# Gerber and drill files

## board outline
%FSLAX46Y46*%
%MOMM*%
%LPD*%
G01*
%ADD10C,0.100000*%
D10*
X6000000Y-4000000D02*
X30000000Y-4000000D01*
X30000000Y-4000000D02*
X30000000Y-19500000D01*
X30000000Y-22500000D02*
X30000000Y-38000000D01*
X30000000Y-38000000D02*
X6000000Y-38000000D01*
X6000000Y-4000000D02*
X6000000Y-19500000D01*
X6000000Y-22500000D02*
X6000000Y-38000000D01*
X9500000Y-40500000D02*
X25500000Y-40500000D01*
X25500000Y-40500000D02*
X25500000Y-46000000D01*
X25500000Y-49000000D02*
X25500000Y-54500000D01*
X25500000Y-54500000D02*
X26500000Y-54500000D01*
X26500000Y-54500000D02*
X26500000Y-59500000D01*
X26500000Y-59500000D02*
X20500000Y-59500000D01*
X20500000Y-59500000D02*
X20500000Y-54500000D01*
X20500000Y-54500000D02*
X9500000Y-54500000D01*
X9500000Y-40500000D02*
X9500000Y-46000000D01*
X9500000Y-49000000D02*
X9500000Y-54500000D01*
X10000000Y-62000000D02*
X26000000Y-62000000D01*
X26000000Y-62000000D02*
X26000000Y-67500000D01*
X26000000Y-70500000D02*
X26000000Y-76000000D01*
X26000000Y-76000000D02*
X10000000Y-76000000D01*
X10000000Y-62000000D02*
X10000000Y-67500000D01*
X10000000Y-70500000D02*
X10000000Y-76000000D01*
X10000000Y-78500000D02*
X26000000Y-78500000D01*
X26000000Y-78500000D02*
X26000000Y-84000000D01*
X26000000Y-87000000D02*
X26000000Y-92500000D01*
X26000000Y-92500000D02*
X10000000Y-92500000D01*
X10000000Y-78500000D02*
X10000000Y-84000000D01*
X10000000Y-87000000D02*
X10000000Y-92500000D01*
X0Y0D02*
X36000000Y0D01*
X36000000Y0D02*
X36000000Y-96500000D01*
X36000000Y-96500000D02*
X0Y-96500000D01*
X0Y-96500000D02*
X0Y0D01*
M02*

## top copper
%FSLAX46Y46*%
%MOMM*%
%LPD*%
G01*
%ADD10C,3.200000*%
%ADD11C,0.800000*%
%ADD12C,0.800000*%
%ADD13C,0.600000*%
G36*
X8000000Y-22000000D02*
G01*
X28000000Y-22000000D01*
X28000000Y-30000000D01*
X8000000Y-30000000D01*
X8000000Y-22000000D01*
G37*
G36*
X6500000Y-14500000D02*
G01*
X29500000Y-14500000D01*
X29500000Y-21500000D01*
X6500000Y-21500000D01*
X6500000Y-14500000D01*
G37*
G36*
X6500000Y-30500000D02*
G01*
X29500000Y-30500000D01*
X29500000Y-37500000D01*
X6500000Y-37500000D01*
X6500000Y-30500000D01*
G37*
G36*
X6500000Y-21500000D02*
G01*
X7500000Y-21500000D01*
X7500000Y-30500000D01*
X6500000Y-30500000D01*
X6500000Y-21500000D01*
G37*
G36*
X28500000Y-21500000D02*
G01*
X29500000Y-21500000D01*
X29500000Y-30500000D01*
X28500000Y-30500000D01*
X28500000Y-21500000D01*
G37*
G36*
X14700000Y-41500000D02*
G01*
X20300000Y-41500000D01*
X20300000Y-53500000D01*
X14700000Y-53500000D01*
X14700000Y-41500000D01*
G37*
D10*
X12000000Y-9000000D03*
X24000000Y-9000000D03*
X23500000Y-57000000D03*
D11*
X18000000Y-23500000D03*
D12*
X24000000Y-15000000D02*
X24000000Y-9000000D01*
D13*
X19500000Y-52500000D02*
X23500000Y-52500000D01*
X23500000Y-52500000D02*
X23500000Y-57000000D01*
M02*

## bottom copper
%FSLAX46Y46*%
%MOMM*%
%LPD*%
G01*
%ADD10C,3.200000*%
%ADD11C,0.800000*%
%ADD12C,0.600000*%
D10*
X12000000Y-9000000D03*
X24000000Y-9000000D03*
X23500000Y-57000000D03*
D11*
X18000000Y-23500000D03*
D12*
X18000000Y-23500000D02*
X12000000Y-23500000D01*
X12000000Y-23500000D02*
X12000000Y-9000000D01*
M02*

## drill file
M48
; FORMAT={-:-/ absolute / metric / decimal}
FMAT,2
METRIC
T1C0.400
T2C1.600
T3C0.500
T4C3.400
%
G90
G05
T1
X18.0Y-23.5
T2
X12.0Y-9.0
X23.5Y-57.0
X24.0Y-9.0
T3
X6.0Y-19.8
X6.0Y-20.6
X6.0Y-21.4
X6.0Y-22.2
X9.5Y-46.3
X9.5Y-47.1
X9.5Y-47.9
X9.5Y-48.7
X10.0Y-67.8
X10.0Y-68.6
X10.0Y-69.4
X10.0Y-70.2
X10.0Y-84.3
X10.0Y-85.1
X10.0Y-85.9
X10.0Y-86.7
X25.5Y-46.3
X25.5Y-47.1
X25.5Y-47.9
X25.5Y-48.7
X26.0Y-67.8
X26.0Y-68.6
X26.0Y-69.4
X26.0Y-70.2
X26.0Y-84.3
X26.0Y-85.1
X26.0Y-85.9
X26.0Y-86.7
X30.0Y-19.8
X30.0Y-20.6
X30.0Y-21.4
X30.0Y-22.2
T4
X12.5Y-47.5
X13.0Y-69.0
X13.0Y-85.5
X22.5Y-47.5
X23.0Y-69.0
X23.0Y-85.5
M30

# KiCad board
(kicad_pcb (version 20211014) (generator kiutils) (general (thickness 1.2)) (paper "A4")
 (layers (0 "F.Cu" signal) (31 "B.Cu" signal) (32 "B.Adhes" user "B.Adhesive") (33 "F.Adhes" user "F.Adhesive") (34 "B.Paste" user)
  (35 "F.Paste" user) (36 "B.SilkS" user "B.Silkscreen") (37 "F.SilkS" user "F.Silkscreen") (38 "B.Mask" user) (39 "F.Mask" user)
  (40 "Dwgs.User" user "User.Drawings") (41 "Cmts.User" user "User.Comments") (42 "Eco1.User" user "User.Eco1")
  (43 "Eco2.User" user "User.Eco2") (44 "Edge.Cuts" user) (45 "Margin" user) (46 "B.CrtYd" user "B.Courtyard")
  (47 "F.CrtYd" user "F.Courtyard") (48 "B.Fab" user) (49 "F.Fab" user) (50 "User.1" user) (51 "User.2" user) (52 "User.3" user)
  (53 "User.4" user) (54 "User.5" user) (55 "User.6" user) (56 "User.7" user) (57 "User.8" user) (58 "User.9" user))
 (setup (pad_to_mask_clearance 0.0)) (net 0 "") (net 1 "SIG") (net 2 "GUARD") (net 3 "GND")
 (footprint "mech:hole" (layer "F.Cu") (at 12.0 9.0)
  (pad "1" thru_hole circle (at 0 0) (size 3.2 3.2) (drill 1.6) (layers *.Cu *.Mask) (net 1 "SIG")))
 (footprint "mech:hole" (layer "F.Cu") (at 24.0 9.0)
  (pad "1" thru_hole circle (at 0 0) (size 3.2 3.2) (drill 1.6) (layers *.Cu *.Mask) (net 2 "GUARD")))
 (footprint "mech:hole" (layer "F.Cu") (at 30.0 19.8) (pad "" np_thru_hole circle (at 0 0) (size 0.5 0.5) (drill 0.5) (layers *.Cu *.Mask)))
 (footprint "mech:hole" (layer "F.Cu") (at 30.0 20.6) (pad "" np_thru_hole circle (at 0 0) (size 0.5 0.5) (drill 0.5) (layers *.Cu *.Mask)))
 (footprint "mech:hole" (layer "F.Cu") (at 30.0 21.400000000000002)
  (pad "" np_thru_hole circle (at 0 0) (size 0.5 0.5) (drill 0.5) (layers *.Cu *.Mask)))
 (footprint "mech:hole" (layer "F.Cu") (at 30.0 22.200000000000003)
  (pad "" np_thru_hole circle (at 0 0) (size 0.5 0.5) (drill 0.5) (layers *.Cu *.Mask)))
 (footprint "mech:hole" (layer "F.Cu") (at 6.0 19.8) (pad "" np_thru_hole circle (at 0 0) (size 0.5 0.5) (drill 0.5) (layers *.Cu *.Mask)))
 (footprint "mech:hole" (layer "F.Cu") (at 6.0 20.6) (pad "" np_thru_hole circle (at 0 0) (size 0.5 0.5) (drill 0.5) (layers *.Cu *.Mask)))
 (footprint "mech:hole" (layer "F.Cu") (at 6.0 21.400000000000002)
  (pad "" np_thru_hole circle (at 0 0) (size 0.5 0.5) (drill 0.5) (layers *.Cu *.Mask)))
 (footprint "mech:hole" (layer "F.Cu") (at 6.0 22.200000000000003)
  (pad "" np_thru_hole circle (at 0 0) (size 0.5 0.5) (drill 0.5) (layers *.Cu *.Mask)))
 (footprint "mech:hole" (layer "F.Cu") (at 12.5 47.5) (pad "" np_thru_hole circle (at 0 0) (size 3.4 3.4) (drill 3.4) (layers *.Cu *.Mask)))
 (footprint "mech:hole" (layer "F.Cu") (at 22.5 47.5) (pad "" np_thru_hole circle (at 0 0) (size 3.4 3.4) (drill 3.4) (layers *.Cu *.Mask)))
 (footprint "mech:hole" (layer "F.Cu") (at 23.5 57.0)
  (pad "1" thru_hole circle (at 0 0) (size 3.2 3.2) (drill 1.6) (layers *.Cu *.Mask) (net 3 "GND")))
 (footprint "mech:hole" (layer "F.Cu") (at 25.5 46.3) (pad "" np_thru_hole circle (at 0 0) (size 0.5 0.5) (drill 0.5) (layers *.Cu *.Mask)))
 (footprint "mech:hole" (layer "F.Cu") (at 25.5 47.099999999999994)
  (pad "" np_thru_hole circle (at 0 0) (size 0.5 0.5) (drill 0.5) (layers *.Cu *.Mask)))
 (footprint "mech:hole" (layer "F.Cu") (at 25.5 47.9) (pad "" np_thru_hole circle (at 0 0) (size 0.5 0.5) (drill 0.5) (layers *.Cu *.Mask)))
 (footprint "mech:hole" (layer "F.Cu") (at 25.5 48.699999999999996)
  (pad "" np_thru_hole circle (at 0 0) (size 0.5 0.5) (drill 0.5) (layers *.Cu *.Mask)))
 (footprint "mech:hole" (layer "F.Cu") (at 9.5 46.3) (pad "" np_thru_hole circle (at 0 0) (size 0.5 0.5) (drill 0.5) (layers *.Cu *.Mask)))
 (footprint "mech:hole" (layer "F.Cu") (at 9.5 47.099999999999994)
  (pad "" np_thru_hole circle (at 0 0) (size 0.5 0.5) (drill 0.5) (layers *.Cu *.Mask)))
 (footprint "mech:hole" (layer "F.Cu") (at 9.5 47.9) (pad "" np_thru_hole circle (at 0 0) (size 0.5 0.5) (drill 0.5) (layers *.Cu *.Mask)))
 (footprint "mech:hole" (layer "F.Cu") (at 9.5 48.699999999999996)
  (pad "" np_thru_hole circle (at 0 0) (size 0.5 0.5) (drill 0.5) (layers *.Cu *.Mask)))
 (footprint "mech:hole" (layer "F.Cu") (at 13.0 69.0) (pad "" np_thru_hole circle (at 0 0) (size 3.4 3.4) (drill 3.4) (layers *.Cu *.Mask)))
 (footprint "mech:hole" (layer "F.Cu") (at 23.0 69.0) (pad "" np_thru_hole circle (at 0 0) (size 3.4 3.4) (drill 3.4) (layers *.Cu *.Mask)))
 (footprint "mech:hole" (layer "F.Cu") (at 26.0 67.8) (pad "" np_thru_hole circle (at 0 0) (size 0.5 0.5) (drill 0.5) (layers *.Cu *.Mask)))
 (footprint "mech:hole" (layer "F.Cu") (at 26.0 68.6) (pad "" np_thru_hole circle (at 0 0) (size 0.5 0.5) (drill 0.5) (layers *.Cu *.Mask)))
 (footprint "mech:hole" (layer "F.Cu") (at 26.0 69.39999999999999)
  (pad "" np_thru_hole circle (at 0 0) (size 0.5 0.5) (drill 0.5) (layers *.Cu *.Mask)))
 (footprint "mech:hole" (layer "F.Cu") (at 26.0 70.2) (pad "" np_thru_hole circle (at 0 0) (size 0.5 0.5) (drill 0.5) (layers *.Cu *.Mask)))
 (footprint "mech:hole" (layer "F.Cu") (at 10.0 67.8) (pad "" np_thru_hole circle (at 0 0) (size 0.5 0.5) (drill 0.5) (layers *.Cu *.Mask)))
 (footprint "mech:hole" (layer "F.Cu") (at 10.0 68.6) (pad "" np_thru_hole circle (at 0 0) (size 0.5 0.5) (drill 0.5) (layers *.Cu *.Mask)))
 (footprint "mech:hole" (layer "F.Cu") (at 10.0 69.39999999999999)
  (pad "" np_thru_hole circle (at 0 0) (size 0.5 0.5) (drill 0.5) (layers *.Cu *.Mask)))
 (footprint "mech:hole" (layer "F.Cu") (at 10.0 70.2) (pad "" np_thru_hole circle (at 0 0) (size 0.5 0.5) (drill 0.5) (layers *.Cu *.Mask)))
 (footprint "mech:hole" (layer "F.Cu") (at 13.0 85.5) (pad "" np_thru_hole circle (at 0 0) (size 3.4 3.4) (drill 3.4) (layers *.Cu *.Mask)))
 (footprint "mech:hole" (layer "F.Cu") (at 23.0 85.5) (pad "" np_thru_hole circle (at 0 0) (size 3.4 3.4) (drill 3.4) (layers *.Cu *.Mask)))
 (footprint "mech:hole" (layer "F.Cu") (at 26.0 84.3) (pad "" np_thru_hole circle (at 0 0) (size 0.5 0.5) (drill 0.5) (layers *.Cu *.Mask)))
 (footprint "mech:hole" (layer "F.Cu") (at 26.0 85.1) (pad "" np_thru_hole circle (at 0 0) (size 0.5 0.5) (drill 0.5) (layers *.Cu *.Mask)))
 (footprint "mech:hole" (layer "F.Cu") (at 26.0 85.89999999999999)
  (pad "" np_thru_hole circle (at 0 0) (size 0.5 0.5) (drill 0.5) (layers *.Cu *.Mask)))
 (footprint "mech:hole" (layer "F.Cu") (at 26.0 86.7) (pad "" np_thru_hole circle (at 0 0) (size 0.5 0.5) (drill 0.5) (layers *.Cu *.Mask)))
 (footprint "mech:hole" (layer "F.Cu") (at 10.0 84.3) (pad "" np_thru_hole circle (at 0 0) (size 0.5 0.5) (drill 0.5) (layers *.Cu *.Mask)))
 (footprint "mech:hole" (layer "F.Cu") (at 10.0 85.1) (pad "" np_thru_hole circle (at 0 0) (size 0.5 0.5) (drill 0.5) (layers *.Cu *.Mask)))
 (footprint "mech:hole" (layer "F.Cu") (at 10.0 85.89999999999999)
  (pad "" np_thru_hole circle (at 0 0) (size 0.5 0.5) (drill 0.5) (layers *.Cu *.Mask)))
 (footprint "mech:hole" (layer "F.Cu") (at 10.0 86.7) (pad "" np_thru_hole circle (at 0 0) (size 0.5 0.5) (drill 0.5) (layers *.Cu *.Mask)))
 (gr_rect (start 8.0 22.0) (end 28.0 30.0) (layer "F.Cu") (width 0) (fill solid))
 (gr_rect (start 6.5 14.5) (end 29.5 21.5) (layer "F.Cu") (width 0) (fill solid))
 (gr_rect (start 6.5 30.5) (end 29.5 37.5) (layer "F.Cu") (width 0) (fill solid))
 (gr_rect (start 6.5 21.5) (end 7.5 30.5) (layer "F.Cu") (width 0) (fill solid))
 (gr_rect (start 28.5 21.5) (end 29.5 30.5) (layer "F.Cu") (width 0) (fill solid))
 (gr_line (start 6.0 4.0) (end 30.0 4.0) (layer "Edge.Cuts") (width 0.1))
 (gr_line (start 30.0 4.0) (end 30.0 19.5) (layer "Edge.Cuts") (width 0.1))
 (gr_line (start 30.0 22.5) (end 30.0 38.0) (layer "Edge.Cuts") (width 0.1))
 (gr_line (start 30.0 38.0) (end 6.0 38.0) (layer "Edge.Cuts") (width 0.1))
 (gr_line (start 6.0 4.0) (end 6.0 19.5) (layer "Edge.Cuts") (width 0.1))
 (gr_line (start 6.0 22.5) (end 6.0 38.0) (layer "Edge.Cuts") (width 0.1))
 (gr_rect (start 14.7 41.5) (end 20.3 53.5) (layer "F.Cu") (width 0) (fill solid))
 (gr_line (start 9.5 40.5) (end 25.5 40.5) (layer "Edge.Cuts") (width 0.1))
 (gr_line (start 25.5 40.5) (end 25.5 46.0) (layer "Edge.Cuts") (width 0.1))
 (gr_line (start 25.5 49.0) (end 25.5 54.5) (layer "Edge.Cuts") (width 0.1))
 (gr_line (start 25.5 54.5) (end 26.5 54.5) (layer "Edge.Cuts") (width 0.1))
 (gr_line (start 26.5 54.5) (end 26.5 59.5) (layer "Edge.Cuts") (width 0.1))
 (gr_line (start 26.5 59.5) (end 20.5 59.5) (layer "Edge.Cuts") (width 0.1))
 (gr_line (start 20.5 59.5) (end 20.5 54.5) (layer "Edge.Cuts") (width 0.1))
 (gr_line (start 20.5 54.5) (end 9.5 54.5) (layer "Edge.Cuts") (width 0.1))
 (gr_line (start 9.5 40.5) (end 9.5 46.0) (layer "Edge.Cuts") (width 0.1))
 (gr_line (start 9.5 49.0) (end 9.5 54.5) (layer "Edge.Cuts") (width 0.1))
 (gr_line (start 10.0 62.0) (end 26.0 62.0) (layer "Edge.Cuts") (width 0.1))
 (gr_line (start 26.0 62.0) (end 26.0 67.5) (layer "Edge.Cuts") (width 0.1))
 (gr_line (start 26.0 70.5) (end 26.0 76.0) (layer "Edge.Cuts") (width 0.1))
 (gr_line (start 26.0 76.0) (end 10.0 76.0) (layer "Edge.Cuts") (width 0.1))
 (gr_line (start 10.0 62.0) (end 10.0 67.5) (layer "Edge.Cuts") (width 0.1))
 (gr_line (start 10.0 70.5) (end 10.0 76.0) (layer "Edge.Cuts") (width 0.1))
 (gr_line (start 10.0 78.5) (end 26.0 78.5) (layer "Edge.Cuts") (width 0.1))
 (gr_line (start 26.0 78.5) (end 26.0 84.0) (layer "Edge.Cuts") (width 0.1))
 (gr_line (start 26.0 87.0) (end 26.0 92.5) (layer "Edge.Cuts") (width 0.1))
 (gr_line (start 26.0 92.5) (end 10.0 92.5) (layer "Edge.Cuts") (width 0.1))
 (gr_line (start 10.0 78.5) (end 10.0 84.0) (layer "Edge.Cuts") (width 0.1))
 (gr_line (start 10.0 87.0) (end 10.0 92.5) (layer "Edge.Cuts") (width 0.1))
 (gr_line (start 0 0) (end 36.0 0) (layer "Edge.Cuts") (width 0.1))
 (gr_line (start 36.0 0) (end 36.0 96.5) (layer "Edge.Cuts") (width 0.1))
 (gr_line (start 36.0 96.5) (end 0 96.5) (layer "Edge.Cuts") (width 0.1))
 (gr_line (start 0 96.5) (end 0 0) (layer "Edge.Cuts") (width 0.1))
 (segment (start 24.0 15.0) (end 24.0 9.0) (width 0.8) (layer "F.Cu") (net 2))
 (via (at 18.0 23.5) (size 0.8) (drill 0.4) (layers "F.Cu" "B.Cu") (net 1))
 (segment (start 18.0 23.5) (end 12.0 23.5) (width 0.6) (layer "B.Cu") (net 1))
 (segment (start 12.0 23.5) (end 12.0 9.0) (width 0.6) (layer "B.Cu") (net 1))
 (segment (start 19.5 52.5) (end 23.5 52.5) (width 0.6) (layer "F.Cu") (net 3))
 (segment (start 23.5 52.5) (end 23.5 57.0) (width 0.6) (layer "F.Cu") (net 3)))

